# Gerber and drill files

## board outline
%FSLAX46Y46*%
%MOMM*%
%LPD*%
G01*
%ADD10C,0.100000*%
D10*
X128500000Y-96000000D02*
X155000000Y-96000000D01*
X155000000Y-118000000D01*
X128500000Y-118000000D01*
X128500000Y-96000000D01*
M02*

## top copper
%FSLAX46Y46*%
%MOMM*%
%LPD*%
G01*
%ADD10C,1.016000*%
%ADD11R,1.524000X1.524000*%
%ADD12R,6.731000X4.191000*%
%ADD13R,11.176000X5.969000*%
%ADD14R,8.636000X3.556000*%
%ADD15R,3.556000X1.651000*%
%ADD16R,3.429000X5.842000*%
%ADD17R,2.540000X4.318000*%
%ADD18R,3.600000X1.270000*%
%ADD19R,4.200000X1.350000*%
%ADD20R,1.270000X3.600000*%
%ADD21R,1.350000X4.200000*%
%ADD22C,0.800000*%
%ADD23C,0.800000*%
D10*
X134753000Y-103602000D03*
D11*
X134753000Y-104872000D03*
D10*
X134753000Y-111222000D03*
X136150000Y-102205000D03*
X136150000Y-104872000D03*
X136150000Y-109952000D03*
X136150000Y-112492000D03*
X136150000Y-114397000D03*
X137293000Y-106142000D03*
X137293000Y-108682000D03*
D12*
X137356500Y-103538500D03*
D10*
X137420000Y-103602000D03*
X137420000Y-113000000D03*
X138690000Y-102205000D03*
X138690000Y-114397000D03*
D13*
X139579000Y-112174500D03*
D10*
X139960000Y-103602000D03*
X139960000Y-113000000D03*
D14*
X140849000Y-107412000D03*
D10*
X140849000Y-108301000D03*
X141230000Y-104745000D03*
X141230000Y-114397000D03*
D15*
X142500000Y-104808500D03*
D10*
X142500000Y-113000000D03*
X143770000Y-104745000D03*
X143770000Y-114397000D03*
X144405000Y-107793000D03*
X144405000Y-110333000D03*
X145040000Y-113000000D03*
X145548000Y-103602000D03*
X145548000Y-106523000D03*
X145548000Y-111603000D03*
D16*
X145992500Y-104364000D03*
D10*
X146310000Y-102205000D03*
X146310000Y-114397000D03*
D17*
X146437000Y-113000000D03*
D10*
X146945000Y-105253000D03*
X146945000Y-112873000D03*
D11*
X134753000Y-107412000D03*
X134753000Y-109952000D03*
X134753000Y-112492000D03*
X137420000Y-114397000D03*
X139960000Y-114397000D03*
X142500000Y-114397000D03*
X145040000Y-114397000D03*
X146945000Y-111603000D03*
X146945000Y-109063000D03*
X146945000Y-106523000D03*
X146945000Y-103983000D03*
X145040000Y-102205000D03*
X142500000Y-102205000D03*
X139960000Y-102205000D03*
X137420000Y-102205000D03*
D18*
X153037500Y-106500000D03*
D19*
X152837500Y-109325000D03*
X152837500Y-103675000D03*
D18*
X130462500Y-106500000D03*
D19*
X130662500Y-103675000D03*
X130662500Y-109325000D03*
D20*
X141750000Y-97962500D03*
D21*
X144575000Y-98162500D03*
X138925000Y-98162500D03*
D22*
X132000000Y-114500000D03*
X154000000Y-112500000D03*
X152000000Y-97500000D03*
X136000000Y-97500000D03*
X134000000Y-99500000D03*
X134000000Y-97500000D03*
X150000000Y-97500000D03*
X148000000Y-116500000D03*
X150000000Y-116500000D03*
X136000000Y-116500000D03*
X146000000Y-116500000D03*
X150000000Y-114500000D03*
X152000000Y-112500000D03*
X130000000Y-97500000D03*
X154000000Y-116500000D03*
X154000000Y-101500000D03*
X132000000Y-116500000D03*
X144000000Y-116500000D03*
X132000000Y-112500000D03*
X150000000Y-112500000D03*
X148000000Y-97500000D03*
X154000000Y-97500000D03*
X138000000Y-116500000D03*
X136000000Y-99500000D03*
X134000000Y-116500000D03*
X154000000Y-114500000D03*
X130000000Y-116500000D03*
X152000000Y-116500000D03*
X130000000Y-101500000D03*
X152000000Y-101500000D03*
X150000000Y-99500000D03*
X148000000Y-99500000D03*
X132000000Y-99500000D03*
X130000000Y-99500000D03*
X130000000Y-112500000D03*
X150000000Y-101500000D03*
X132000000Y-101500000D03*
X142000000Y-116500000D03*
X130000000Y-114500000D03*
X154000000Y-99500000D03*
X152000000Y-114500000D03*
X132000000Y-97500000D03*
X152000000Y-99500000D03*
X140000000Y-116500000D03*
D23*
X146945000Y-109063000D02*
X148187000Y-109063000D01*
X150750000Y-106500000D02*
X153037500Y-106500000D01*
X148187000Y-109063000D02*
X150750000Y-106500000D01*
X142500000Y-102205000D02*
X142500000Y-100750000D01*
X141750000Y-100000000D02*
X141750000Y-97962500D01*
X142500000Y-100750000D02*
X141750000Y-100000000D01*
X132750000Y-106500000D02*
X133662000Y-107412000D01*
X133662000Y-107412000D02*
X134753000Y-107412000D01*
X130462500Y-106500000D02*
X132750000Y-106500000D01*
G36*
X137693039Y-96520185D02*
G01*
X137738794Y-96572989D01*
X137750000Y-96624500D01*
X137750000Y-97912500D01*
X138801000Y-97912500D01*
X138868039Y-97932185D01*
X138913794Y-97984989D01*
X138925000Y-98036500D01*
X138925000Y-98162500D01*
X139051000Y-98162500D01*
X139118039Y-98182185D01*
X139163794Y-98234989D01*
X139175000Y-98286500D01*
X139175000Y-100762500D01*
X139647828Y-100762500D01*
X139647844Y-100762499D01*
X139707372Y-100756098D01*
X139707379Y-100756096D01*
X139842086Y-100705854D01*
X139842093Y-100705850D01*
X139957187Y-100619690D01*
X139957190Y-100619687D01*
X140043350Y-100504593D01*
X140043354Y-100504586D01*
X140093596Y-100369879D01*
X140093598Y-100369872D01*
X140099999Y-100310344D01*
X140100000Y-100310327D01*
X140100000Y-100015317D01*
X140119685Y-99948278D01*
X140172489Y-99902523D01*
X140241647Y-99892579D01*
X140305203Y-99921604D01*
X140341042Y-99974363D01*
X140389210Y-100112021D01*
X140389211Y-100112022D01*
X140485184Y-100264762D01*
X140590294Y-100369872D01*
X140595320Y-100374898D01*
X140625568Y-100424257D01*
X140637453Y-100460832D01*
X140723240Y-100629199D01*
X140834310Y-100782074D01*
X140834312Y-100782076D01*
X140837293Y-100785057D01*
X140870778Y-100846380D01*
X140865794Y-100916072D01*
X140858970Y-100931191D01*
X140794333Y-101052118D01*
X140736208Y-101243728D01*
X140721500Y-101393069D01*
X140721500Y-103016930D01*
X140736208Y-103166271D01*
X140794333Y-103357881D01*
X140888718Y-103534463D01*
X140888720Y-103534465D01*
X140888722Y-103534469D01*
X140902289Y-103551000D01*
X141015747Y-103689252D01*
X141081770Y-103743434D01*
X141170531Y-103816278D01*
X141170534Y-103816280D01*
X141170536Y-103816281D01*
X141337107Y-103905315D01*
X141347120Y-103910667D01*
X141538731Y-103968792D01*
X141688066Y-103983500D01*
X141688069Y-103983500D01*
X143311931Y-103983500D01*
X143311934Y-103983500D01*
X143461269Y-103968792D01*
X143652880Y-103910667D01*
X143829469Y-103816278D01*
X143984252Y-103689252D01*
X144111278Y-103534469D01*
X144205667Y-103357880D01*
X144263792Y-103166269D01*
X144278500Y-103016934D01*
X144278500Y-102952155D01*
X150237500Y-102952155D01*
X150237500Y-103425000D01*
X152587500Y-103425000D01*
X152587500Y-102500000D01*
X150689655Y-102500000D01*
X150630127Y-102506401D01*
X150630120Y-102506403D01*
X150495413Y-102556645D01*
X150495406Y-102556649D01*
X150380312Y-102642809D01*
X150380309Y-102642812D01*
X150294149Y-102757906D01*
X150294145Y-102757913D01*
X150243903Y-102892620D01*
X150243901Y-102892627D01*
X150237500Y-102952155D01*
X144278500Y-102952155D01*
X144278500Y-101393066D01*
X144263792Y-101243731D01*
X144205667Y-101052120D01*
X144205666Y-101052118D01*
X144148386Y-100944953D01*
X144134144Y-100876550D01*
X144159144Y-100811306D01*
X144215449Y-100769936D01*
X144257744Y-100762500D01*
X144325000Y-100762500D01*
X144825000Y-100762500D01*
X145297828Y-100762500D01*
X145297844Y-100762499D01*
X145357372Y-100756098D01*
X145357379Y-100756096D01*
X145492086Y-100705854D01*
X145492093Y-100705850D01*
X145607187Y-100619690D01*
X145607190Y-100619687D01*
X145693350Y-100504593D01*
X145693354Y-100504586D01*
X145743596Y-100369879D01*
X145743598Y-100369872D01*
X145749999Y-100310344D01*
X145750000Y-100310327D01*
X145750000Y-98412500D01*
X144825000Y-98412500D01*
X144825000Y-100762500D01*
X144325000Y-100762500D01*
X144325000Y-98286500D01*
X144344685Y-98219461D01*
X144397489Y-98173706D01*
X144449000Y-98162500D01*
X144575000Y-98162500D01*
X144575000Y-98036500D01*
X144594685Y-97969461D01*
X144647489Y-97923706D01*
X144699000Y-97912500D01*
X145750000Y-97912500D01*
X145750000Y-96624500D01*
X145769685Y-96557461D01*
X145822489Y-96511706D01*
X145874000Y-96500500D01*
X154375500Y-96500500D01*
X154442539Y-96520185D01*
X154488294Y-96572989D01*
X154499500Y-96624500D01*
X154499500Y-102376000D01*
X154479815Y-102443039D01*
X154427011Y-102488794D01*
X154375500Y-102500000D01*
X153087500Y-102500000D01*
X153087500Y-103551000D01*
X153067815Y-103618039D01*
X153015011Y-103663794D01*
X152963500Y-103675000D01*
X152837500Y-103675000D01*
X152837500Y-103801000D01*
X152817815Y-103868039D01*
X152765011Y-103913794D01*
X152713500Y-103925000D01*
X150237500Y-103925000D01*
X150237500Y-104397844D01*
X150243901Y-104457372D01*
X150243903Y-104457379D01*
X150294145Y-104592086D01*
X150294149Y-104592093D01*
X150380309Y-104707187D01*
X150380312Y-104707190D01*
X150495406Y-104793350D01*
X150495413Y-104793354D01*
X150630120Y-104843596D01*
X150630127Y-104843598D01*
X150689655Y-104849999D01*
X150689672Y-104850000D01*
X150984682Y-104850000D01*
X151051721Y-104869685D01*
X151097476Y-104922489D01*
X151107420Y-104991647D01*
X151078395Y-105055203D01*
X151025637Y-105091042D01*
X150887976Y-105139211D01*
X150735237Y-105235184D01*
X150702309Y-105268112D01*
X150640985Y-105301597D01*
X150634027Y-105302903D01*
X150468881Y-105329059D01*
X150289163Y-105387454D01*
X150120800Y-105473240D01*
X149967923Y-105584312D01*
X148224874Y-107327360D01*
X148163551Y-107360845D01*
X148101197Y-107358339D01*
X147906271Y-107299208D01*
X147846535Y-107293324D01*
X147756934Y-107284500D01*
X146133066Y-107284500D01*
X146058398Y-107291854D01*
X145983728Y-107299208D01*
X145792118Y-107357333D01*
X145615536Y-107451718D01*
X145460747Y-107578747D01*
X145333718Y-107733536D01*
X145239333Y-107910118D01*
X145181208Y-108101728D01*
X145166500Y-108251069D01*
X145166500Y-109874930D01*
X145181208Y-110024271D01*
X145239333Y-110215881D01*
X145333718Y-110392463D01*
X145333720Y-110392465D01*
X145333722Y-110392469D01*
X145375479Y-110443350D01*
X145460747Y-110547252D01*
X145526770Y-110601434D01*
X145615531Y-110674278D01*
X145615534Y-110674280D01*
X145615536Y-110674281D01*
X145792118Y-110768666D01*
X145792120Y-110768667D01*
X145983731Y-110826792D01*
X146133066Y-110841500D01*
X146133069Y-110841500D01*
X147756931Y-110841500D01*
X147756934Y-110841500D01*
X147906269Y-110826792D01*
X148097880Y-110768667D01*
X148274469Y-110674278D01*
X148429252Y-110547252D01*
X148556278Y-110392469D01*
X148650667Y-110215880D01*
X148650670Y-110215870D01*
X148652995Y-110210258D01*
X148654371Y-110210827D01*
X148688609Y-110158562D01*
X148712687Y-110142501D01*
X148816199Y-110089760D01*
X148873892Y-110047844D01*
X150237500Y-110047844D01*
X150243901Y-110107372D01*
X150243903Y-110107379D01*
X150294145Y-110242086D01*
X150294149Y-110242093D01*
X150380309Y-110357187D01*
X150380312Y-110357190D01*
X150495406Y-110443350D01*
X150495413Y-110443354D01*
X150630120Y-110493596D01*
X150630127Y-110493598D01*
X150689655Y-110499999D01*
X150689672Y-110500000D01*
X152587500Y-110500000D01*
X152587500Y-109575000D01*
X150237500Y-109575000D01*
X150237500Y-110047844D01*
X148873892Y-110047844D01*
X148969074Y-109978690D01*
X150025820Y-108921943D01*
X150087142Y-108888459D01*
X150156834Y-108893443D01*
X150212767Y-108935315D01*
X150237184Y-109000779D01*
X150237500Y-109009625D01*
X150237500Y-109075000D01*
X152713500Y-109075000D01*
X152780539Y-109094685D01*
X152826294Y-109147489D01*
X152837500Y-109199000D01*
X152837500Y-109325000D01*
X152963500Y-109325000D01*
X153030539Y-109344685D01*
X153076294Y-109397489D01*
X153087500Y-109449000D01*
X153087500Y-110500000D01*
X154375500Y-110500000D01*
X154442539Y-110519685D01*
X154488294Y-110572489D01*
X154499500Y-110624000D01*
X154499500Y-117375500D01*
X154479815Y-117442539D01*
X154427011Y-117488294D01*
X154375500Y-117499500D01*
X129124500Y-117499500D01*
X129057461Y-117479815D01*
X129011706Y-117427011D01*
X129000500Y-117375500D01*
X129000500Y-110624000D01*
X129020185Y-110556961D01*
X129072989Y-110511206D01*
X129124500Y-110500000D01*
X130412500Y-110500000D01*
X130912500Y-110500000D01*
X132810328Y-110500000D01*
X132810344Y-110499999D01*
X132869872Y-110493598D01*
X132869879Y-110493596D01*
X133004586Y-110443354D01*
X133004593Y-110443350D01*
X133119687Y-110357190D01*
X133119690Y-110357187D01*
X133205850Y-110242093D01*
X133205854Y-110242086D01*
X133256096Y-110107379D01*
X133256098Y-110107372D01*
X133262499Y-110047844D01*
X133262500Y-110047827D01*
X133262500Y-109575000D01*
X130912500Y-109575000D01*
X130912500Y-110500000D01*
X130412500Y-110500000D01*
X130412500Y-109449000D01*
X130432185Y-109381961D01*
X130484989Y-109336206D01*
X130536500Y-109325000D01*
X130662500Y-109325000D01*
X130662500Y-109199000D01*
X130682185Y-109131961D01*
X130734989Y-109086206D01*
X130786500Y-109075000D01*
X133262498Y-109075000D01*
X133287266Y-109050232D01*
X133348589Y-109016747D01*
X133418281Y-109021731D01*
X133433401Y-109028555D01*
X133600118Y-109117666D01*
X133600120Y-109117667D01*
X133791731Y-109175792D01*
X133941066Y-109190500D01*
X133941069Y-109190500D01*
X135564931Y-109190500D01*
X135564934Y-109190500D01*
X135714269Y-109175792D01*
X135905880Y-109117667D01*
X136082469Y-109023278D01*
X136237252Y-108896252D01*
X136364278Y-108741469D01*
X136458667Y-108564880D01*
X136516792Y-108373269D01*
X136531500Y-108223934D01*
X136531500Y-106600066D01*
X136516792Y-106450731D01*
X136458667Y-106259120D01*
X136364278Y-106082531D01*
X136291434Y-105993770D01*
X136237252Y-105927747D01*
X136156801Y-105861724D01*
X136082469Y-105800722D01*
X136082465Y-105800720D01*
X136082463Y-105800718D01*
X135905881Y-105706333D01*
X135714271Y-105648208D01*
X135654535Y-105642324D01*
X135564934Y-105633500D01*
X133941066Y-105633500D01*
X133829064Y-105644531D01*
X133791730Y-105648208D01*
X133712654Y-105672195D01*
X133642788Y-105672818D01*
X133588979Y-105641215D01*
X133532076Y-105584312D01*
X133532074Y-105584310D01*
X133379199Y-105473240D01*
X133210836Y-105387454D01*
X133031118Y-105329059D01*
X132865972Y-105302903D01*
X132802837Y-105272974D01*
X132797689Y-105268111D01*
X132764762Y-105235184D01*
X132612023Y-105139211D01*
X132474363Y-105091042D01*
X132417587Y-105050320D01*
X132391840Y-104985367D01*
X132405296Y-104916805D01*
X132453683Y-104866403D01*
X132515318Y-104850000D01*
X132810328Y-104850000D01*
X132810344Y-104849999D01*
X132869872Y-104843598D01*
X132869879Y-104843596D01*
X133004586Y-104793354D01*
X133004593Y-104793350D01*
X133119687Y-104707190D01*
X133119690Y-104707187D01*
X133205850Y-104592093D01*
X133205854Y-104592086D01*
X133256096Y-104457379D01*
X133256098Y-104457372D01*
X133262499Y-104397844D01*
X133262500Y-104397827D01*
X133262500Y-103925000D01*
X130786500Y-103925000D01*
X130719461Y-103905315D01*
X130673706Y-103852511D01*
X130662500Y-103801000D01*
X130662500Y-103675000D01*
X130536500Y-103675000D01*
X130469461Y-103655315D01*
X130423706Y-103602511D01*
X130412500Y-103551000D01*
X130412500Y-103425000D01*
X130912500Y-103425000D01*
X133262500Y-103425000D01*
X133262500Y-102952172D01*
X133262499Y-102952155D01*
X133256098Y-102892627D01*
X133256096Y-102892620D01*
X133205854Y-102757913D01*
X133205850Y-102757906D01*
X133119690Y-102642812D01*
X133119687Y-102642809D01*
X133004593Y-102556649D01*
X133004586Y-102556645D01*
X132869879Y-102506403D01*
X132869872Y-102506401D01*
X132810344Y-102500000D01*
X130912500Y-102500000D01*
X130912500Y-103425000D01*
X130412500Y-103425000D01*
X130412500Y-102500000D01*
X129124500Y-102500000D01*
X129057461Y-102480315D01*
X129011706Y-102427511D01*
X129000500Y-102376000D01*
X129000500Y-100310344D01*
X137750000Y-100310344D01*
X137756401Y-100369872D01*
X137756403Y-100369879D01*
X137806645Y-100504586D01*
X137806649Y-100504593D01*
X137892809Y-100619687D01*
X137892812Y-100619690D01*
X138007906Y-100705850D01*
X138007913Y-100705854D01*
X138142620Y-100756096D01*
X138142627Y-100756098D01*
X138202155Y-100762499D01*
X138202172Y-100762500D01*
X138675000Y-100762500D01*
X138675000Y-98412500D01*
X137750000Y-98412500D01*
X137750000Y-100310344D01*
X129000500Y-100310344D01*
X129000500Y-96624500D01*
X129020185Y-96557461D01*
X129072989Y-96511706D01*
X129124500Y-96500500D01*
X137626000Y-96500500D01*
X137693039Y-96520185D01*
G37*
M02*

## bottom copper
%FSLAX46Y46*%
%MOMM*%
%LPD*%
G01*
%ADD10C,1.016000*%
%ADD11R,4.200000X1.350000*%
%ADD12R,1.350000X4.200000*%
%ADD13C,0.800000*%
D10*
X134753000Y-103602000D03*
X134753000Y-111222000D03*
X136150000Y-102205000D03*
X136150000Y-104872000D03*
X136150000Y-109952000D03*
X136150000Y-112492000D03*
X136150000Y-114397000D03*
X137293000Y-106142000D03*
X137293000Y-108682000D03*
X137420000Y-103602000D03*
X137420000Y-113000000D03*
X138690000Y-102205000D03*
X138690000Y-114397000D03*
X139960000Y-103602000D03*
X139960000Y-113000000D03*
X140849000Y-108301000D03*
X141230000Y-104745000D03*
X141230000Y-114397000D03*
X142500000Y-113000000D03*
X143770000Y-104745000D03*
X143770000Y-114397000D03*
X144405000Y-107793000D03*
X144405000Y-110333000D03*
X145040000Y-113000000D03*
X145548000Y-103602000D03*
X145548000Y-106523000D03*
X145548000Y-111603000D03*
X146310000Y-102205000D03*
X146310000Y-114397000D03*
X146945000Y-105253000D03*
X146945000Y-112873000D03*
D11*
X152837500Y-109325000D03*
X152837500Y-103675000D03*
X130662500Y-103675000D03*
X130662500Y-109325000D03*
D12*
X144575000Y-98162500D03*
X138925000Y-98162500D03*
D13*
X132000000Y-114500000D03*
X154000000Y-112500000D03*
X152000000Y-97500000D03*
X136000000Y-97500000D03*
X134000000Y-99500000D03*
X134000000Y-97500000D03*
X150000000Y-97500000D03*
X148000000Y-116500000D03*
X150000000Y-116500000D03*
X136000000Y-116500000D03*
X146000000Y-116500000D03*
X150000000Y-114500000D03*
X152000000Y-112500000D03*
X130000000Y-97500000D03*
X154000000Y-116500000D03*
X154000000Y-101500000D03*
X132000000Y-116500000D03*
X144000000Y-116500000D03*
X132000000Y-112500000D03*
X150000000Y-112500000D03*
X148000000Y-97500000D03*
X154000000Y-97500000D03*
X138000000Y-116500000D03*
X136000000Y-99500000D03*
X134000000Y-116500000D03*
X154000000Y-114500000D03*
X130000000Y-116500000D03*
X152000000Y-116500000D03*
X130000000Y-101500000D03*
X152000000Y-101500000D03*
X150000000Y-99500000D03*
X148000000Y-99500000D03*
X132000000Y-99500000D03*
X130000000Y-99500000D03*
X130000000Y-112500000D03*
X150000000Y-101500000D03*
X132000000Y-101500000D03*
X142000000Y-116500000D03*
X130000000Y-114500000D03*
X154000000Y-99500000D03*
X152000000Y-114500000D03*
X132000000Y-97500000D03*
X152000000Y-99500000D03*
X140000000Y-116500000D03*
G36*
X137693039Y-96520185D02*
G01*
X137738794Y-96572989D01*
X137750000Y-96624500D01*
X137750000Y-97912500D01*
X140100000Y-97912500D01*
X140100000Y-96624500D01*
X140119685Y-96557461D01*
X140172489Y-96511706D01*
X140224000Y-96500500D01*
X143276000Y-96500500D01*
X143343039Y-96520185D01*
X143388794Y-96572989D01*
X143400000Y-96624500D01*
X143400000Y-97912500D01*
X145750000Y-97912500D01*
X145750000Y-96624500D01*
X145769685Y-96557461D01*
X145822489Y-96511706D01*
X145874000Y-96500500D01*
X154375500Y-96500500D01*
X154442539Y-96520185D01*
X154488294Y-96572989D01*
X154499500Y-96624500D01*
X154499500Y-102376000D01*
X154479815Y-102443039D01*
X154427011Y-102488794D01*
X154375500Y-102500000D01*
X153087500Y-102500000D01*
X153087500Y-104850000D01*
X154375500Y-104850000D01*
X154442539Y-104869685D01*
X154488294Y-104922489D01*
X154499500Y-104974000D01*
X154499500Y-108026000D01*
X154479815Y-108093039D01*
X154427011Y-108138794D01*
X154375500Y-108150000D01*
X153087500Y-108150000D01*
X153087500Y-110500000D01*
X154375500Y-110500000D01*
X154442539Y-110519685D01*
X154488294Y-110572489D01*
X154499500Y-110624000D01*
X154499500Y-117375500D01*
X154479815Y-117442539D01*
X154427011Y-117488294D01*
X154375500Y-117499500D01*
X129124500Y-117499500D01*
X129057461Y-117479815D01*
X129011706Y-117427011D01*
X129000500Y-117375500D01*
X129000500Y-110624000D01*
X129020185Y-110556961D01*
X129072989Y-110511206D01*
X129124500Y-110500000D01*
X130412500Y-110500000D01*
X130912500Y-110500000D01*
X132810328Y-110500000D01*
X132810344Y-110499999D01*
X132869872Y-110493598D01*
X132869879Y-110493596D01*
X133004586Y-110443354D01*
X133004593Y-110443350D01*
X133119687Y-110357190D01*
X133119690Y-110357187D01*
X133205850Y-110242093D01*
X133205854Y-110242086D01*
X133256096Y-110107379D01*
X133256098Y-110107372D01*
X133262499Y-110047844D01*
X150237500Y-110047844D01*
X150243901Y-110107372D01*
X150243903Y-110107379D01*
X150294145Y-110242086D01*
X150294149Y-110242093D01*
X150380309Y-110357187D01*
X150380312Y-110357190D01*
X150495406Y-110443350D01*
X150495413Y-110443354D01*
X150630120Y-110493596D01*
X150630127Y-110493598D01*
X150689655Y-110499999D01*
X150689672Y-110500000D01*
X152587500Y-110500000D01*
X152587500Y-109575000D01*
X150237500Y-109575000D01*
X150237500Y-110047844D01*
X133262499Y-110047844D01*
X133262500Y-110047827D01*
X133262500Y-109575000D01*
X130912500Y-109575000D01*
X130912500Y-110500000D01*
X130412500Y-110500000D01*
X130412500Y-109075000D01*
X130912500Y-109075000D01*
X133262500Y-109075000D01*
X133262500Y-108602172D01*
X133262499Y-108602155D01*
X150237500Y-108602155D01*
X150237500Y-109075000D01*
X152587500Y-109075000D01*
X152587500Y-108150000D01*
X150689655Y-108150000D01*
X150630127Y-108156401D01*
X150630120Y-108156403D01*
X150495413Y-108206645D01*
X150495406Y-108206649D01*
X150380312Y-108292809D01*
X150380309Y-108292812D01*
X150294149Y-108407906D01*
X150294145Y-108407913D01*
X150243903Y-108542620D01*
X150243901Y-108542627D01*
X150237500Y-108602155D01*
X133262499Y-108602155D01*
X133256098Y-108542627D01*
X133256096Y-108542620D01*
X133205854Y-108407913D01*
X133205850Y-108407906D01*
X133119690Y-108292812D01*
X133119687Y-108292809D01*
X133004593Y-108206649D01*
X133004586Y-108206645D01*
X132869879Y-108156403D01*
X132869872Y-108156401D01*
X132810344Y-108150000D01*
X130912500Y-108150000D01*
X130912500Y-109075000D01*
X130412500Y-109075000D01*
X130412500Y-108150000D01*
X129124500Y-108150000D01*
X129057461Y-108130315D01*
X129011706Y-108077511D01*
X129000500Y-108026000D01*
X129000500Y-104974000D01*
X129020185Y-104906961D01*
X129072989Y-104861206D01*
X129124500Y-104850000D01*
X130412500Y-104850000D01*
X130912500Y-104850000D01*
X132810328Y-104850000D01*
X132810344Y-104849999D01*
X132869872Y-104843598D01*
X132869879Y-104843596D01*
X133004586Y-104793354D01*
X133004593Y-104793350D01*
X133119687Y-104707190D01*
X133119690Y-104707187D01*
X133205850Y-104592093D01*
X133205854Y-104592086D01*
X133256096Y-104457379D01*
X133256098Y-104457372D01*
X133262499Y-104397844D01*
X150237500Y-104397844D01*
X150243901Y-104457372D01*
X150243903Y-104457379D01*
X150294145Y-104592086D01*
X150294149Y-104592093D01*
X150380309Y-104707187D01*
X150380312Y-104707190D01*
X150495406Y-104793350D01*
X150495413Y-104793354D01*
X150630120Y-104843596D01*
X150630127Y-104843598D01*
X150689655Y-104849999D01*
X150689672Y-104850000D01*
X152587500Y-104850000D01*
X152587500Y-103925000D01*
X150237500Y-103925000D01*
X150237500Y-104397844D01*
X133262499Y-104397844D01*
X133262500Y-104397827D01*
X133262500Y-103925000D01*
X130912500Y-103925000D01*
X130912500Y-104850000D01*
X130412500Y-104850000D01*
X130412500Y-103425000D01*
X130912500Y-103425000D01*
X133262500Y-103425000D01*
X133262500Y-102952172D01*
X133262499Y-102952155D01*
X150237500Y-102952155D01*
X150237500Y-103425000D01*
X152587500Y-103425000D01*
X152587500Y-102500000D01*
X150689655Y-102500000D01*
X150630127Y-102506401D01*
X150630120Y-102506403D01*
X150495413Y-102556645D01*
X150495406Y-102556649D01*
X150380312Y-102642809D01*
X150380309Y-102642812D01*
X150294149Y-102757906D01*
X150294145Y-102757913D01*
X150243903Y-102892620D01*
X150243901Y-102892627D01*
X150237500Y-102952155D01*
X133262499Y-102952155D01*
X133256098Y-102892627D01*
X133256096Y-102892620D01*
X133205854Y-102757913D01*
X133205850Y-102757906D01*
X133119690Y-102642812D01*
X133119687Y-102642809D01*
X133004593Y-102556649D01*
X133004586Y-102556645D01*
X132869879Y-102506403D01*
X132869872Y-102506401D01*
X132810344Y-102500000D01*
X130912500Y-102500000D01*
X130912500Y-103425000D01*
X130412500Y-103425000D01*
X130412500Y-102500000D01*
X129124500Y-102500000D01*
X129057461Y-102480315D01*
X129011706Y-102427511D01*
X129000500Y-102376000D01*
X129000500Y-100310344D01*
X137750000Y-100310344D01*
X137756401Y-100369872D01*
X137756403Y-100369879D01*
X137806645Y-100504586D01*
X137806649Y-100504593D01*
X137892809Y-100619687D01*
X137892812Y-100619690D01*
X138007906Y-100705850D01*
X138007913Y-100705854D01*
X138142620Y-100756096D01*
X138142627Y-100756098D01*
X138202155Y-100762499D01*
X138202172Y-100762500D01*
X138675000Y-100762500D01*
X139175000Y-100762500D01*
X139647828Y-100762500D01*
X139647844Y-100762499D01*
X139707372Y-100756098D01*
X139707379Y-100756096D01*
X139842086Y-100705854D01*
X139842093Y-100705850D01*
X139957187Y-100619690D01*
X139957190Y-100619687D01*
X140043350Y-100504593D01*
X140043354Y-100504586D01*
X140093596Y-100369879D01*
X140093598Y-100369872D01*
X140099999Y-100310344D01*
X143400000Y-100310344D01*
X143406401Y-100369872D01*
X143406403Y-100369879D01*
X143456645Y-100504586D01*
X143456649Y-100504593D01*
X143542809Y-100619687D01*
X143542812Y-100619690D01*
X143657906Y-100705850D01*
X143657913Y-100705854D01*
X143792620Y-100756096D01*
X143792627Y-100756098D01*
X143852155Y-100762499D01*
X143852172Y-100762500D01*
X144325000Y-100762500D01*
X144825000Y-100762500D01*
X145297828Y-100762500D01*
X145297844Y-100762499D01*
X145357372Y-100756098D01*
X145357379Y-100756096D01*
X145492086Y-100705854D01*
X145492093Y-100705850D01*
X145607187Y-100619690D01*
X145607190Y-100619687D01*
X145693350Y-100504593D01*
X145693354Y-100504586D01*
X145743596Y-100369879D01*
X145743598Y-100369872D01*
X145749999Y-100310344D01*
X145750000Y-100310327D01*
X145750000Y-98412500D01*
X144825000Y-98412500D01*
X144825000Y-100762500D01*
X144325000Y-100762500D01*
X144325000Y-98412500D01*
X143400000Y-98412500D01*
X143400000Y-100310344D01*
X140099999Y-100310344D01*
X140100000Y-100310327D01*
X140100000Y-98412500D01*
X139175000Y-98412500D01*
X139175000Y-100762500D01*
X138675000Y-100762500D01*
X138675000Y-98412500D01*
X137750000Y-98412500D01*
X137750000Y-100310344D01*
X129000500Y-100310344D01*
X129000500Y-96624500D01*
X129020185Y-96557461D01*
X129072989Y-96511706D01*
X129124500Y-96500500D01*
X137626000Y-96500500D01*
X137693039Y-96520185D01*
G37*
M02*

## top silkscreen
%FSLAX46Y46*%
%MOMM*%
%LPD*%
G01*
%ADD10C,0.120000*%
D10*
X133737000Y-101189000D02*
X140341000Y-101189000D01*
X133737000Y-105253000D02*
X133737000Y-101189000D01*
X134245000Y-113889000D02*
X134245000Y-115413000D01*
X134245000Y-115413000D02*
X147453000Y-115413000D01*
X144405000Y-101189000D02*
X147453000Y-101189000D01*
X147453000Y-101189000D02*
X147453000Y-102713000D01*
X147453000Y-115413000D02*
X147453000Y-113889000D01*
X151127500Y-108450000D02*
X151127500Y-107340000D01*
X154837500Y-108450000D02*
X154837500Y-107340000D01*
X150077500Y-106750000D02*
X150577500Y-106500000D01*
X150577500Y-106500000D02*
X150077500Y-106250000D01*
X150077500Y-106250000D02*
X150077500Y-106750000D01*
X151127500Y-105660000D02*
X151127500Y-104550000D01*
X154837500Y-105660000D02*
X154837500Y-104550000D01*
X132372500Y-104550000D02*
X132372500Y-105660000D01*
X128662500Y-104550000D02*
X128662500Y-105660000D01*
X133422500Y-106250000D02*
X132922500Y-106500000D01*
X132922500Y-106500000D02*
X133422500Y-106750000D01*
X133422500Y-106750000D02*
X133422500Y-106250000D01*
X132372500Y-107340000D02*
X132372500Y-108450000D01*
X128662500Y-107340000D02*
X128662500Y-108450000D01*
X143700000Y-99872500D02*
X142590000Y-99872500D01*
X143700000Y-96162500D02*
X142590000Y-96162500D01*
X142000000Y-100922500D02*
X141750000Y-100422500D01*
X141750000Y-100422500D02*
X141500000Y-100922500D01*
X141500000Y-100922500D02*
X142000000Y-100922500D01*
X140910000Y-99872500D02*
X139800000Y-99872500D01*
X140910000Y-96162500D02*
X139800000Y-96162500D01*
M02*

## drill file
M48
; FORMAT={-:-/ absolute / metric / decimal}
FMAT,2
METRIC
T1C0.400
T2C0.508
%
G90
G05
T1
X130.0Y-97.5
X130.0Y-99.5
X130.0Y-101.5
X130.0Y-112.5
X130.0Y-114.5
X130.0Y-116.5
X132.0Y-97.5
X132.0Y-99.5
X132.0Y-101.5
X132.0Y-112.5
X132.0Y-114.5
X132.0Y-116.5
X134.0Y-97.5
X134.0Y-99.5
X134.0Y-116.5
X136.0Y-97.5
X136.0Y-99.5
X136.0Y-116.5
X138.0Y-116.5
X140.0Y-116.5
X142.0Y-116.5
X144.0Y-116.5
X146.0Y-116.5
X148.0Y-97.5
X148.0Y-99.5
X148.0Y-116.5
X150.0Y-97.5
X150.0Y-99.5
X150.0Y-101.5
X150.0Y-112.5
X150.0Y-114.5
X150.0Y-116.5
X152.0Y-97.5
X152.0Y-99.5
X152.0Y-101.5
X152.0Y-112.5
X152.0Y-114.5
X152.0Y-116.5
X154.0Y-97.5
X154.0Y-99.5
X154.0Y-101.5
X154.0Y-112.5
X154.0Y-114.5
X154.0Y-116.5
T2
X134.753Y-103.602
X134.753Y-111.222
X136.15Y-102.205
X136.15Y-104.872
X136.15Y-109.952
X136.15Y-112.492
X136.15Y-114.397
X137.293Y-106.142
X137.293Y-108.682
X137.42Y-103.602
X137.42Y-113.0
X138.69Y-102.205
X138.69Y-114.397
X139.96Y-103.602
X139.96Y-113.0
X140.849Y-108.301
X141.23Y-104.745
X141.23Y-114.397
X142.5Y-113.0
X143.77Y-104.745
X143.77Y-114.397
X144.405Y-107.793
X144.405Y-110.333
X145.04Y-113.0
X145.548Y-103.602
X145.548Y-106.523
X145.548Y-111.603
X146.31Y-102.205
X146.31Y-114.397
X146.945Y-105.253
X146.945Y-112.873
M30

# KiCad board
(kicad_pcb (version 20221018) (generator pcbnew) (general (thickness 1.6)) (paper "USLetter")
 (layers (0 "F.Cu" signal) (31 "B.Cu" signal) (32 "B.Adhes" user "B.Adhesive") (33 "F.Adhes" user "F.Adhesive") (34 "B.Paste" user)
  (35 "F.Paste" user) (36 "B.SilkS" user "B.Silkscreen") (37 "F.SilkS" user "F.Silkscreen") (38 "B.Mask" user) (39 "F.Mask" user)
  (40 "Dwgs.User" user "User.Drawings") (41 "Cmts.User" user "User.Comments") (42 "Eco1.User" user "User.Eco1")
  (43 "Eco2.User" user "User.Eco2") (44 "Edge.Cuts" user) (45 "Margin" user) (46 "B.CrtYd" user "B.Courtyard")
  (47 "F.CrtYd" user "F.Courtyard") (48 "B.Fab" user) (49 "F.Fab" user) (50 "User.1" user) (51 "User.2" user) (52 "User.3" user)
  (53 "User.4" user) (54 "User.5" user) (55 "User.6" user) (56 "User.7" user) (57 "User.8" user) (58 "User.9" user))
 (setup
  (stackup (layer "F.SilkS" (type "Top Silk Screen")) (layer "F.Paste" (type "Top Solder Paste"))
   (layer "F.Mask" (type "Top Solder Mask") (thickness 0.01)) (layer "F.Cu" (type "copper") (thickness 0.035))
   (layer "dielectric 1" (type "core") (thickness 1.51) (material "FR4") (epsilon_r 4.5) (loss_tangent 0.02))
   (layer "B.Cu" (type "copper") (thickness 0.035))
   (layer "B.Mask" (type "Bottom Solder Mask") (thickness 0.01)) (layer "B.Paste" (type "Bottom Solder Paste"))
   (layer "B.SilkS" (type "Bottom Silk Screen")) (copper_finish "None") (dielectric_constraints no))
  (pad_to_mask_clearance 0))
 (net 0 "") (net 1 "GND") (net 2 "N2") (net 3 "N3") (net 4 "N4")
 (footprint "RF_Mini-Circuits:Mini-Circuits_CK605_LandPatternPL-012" (layer "F.Cu") (at 140.849 108.301)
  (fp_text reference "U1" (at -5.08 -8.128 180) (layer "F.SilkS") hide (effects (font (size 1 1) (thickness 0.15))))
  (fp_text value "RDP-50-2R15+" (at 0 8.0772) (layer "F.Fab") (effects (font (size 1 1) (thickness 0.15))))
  (fp_line (start -7.112 -7.112) (end -0.508 -7.112) (stroke (width 0.12) (type solid)) (layer "F.SilkS"))
  (fp_line (start -7.112 -3.048) (end -7.112 -7.112) (stroke (width 0.12) (type solid)) (layer "F.SilkS"))
  (fp_line (start -6.604 5.588) (end -6.604 7.112) (stroke (width 0.12) (type solid)) (layer "F.SilkS"))
  (fp_line (start -6.604 7.112) (end 6.604 7.112) (stroke (width 0.12) (type solid)) (layer "F.SilkS"))
  (fp_line (start 3.556 -7.112) (end 6.604 -7.112) (stroke (width 0.12) (type solid)) (layer "F.SilkS"))
  (fp_line (start 6.604 -7.112) (end 6.604 -5.588) (stroke (width 0.12) (type solid)) (layer "F.SilkS"))
  (fp_line (start 6.604 7.112) (end 6.604 5.588) (stroke (width 0.12) (type solid)) (layer "F.SilkS"))
  (pad "1" thru_hole circle (at -6.096 -4.699) (size 1.016 1.016) (drill 0.508) (layers "*.Cu") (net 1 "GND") (zone_connect 2))
  (pad "1" smd rect (at -6.096 -3.429 270) (size 1.524 1.524) (layers "F.Cu" "F.Paste" "F.Mask") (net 1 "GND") (zone_connect 2))
  (pad "1" thru_hole circle (at -6.096 2.921) (size 1.016 1.016) (drill 0.508) (layers "*.Cu") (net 1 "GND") (zone_connect 2))
  (pad "1" thru_hole circle (at -4.699 -6.096) (size 1.016 1.016) (drill 0.508) (layers "*.Cu") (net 1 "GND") (zone_connect 2))
  (pad "1" thru_hole circle (at -4.699 -3.429) (size 1.016 1.016) (drill 0.508) (layers "*.Cu") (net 1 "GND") (zone_connect 2))
  (pad "1" thru_hole circle (at -4.699 1.651) (size 1.016 1.016) (drill 0.508) (layers "*.Cu") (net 1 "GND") (zone_connect 2))
  (pad "1" thru_hole circle (at -4.699 4.191) (size 1.016 1.016) (drill 0.508) (layers "*.Cu") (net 1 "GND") (zone_connect 2))
  (pad "1" thru_hole circle (at -4.699 6.096) (size 1.016 1.016) (drill 0.508) (layers "*.Cu") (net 1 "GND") (zone_connect 2))
  (pad "1" thru_hole circle (at -3.556 -2.159) (size 1.016 1.016) (drill 0.508) (layers "*.Cu") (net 1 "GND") (zone_connect 2))
  (pad "1" thru_hole circle (at -3.556 0.381) (size 1.016 1.016) (drill 0.508) (layers "*.Cu") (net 1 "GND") (zone_connect 2))
  (pad "1" smd rect (at -3.4925 -4.7625) (size 6.731 4.191) (layers "F.Cu") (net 1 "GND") (zone_connect 2))
  (pad "1" thru_hole circle (at -3.429 -4.699) (size 1.016 1.016) (drill 0.508) (layers "*.Cu") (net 1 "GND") (zone_connect 2))
  (pad "1" thru_hole circle (at -3.429 4.699) (size 1.016 1.016) (drill 0.508) (layers "*.Cu") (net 1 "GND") (zone_connect 2))
  (pad "1" thru_hole circle (at -2.159 -6.096) (size 1.016 1.016) (drill 0.508) (layers "*.Cu") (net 1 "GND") (zone_connect 2))
  (pad "1" thru_hole circle (at -2.159 6.096) (size 1.016 1.016) (drill 0.508) (layers "*.Cu") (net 1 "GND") (zone_connect 2))
  (pad "1" smd rect (at -1.27 3.8735) (size 11.176 5.969) (layers "F.Cu") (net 1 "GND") (zone_connect 2))
  (pad "1" thru_hole circle (at -0.889 -4.699) (size 1.016 1.016) (drill 0.508) (layers "*.Cu") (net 1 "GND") (zone_connect 2))
  (pad "1" thru_hole circle (at -0.889 4.699) (size 1.016 1.016) (drill 0.508) (layers "*.Cu") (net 1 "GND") (zone_connect 2))
  (pad "1" smd rect (at 0 -0.889) (size 8.636 3.556) (layers "F.Cu") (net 1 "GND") (zone_connect 2))
  (pad "1" thru_hole circle (at 0 0) (size 1.016 1.016) (drill 0.508) (layers "*.Cu") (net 1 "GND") (zone_connect 2))
  (pad "1" thru_hole circle (at 0.381 -3.556) (size 1.016 1.016) (drill 0.508) (layers "*.Cu") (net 1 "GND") (zone_connect 2))
  (pad "1" thru_hole circle (at 0.381 6.096) (size 1.016 1.016) (drill 0.508) (layers "*.Cu") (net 1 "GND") (zone_connect 2))
  (pad "1" smd rect (at 1.651 -3.4925) (size 3.556 1.651) (layers "F.Cu") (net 1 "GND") (zone_connect 2))
  (pad "1" thru_hole circle (at 1.651 4.699) (size 1.016 1.016) (drill 0.508) (layers "*.Cu") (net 1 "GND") (zone_connect 2))
  (pad "1" thru_hole circle (at 2.921 -3.556) (size 1.016 1.016) (drill 0.508) (layers "*.Cu") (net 1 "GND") (zone_connect 2))
  (pad "1" thru_hole circle (at 2.921 6.096) (size 1.016 1.016) (drill 0.508) (layers "*.Cu") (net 1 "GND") (zone_connect 2))
  (pad "1" thru_hole circle (at 3.556 -0.508) (size 1.016 1.016) (drill 0.508) (layers "*.Cu") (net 1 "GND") (zone_connect 2))
  (pad "1" thru_hole circle (at 3.556 2.032) (size 1.016 1.016) (drill 0.508) (layers "*.Cu") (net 1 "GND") (zone_connect 2))
  (pad "1" thru_hole circle (at 4.191 4.699) (size 1.016 1.016) (drill 0.508) (layers "*.Cu") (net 1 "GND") (zone_connect 2))
  (pad "1" thru_hole circle (at 4.699 -4.699) (size 1.016 1.016) (drill 0.508) (layers "*.Cu") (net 1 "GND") (zone_connect 2))
  (pad "1" thru_hole circle (at 4.699 -1.778) (size 1.016 1.016) (drill 0.508) (layers "*.Cu") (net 1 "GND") (zone_connect 2))
  (pad "1" thru_hole circle (at 4.699 3.302) (size 1.016 1.016) (drill 0.508) (layers "*.Cu") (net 1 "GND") (zone_connect 2))
  (pad "1" smd rect (at 5.1435 -3.937) (size 3.429 5.842) (layers "F.Cu") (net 1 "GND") (zone_connect 2))
  (pad "1" thru_hole circle (at 5.461 -6.096) (size 1.016 1.016) (drill 0.508) (layers "*.Cu") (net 1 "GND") (zone_connect 2))
  (pad "1" thru_hole circle (at 5.461 6.096) (size 1.016 1.016) (drill 0.508) (layers "*.Cu") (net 1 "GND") (zone_connect 2))
  (pad "1" smd rect (at 5.588 4.699) (size 2.54 4.318) (layers "F.Cu") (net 1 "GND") (zone_connect 2))
  (pad "1" thru_hole circle (at 6.096 -3.048) (size 1.016 1.016) (drill 0.508) (layers "*.Cu") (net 1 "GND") (zone_connect 2))
  (pad "1" thru_hole circle (at 6.096 4.572) (size 1.016 1.016) (drill 0.508) (layers "*.Cu") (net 1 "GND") (zone_connect 2))
  (pad "2" smd rect (at -6.096 -0.889 270) (size 1.524 1.524) (layers "F.Cu" "F.Paste" "F.Mask") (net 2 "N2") (clearance 1.016))
  (pad "3" smd rect (at -6.096 1.651 270) (size 1.524 1.524) (layers "F.Cu" "F.Paste" "F.Mask") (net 1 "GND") (zone_connect 2))
  (pad "4" smd rect (at -6.096 4.191 270) (size 1.524 1.524) (layers "F.Cu" "F.Paste" "F.Mask") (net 1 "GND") (zone_connect 2))
  (pad "5" smd rect (at -3.429 6.096 270) (size 1.524 1.524) (layers "F.Cu" "F.Paste" "F.Mask") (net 1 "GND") (zone_connect 2))
  (pad "6" smd rect (at -0.889 6.096 270) (size 1.524 1.524) (layers "F.Cu" "F.Paste" "F.Mask") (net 1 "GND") (zone_connect 2))
  (pad "7" smd rect (at 1.651 6.096 270) (size 1.524 1.524) (layers "F.Cu" "F.Paste" "F.Mask") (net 1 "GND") (zone_connect 2))
  (pad "8" smd rect (at 4.191 6.096 270) (size 1.524 1.524) (layers "F.Cu" "F.Paste" "F.Mask") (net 1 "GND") (zone_connect 2))
  (pad "9" smd rect (at 6.096 3.302 270) (size 1.524 1.524) (layers "F.Cu" "F.Paste" "F.Mask") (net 1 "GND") (zone_connect 2))
  (pad "10" smd rect (at 6.096 0.762 270) (size 1.524 1.524) (layers "F.Cu" "F.Paste" "F.Mask") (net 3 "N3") (clearance 1.016))
  (pad "11" smd rect (at 6.096 -1.778 270) (size 1.524 1.524) (layers "F.Cu" "F.Paste" "F.Mask") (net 1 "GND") (zone_connect 2))
  (pad "12" smd rect (at 6.096 -4.318 270) (size 1.524 1.524) (layers "F.Cu" "F.Paste" "F.Mask") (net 1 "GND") (zone_connect 2))
  (pad "13" smd rect (at 4.191 -6.096 270) (size 1.524 1.524) (layers "F.Cu" "F.Paste" "F.Mask") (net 1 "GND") (zone_connect 2))
  (pad "14" smd rect (at 1.651 -6.096 270) (size 1.524 1.524) (layers "F.Cu" "F.Paste" "F.Mask") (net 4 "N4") (clearance 1.016))
  (pad "15" smd rect (at -0.889 -6.096 270) (size 1.524 1.524) (layers "F.Cu" "F.Paste" "F.Mask") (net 1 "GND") (zone_connect 2))
  (pad "16" smd rect (at -3.429 -6.096 270) (size 1.524 1.524) (layers "F.Cu" "F.Paste" "F.Mask") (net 1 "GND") (zone_connect 2)))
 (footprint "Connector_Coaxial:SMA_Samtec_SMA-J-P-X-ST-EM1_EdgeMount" (layer "F.Cu") (at 152.8375 106.5 90)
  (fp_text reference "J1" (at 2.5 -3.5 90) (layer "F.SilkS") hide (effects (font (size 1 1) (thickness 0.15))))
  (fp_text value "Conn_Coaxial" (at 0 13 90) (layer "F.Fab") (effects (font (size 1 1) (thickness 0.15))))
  (fp_line (start -1.95 -1.71) (end -0.84 -1.71) (stroke (width 0.12) (type solid)) (layer "F.SilkS"))
  (fp_line (start -1.95 2) (end -0.84 2) (stroke (width 0.12) (type solid)) (layer "F.SilkS"))
  (fp_line (start -0.25 -2.76) (end 0 -2.26) (stroke (width 0.12) (type solid)) (layer "F.SilkS"))
  (fp_line (start 0 -2.26) (end 0.25 -2.76) (stroke (width 0.12) (type solid)) (layer "F.SilkS"))
  (fp_line (start 0.25 -2.76) (end -0.25 -2.76) (stroke (width 0.12) (type solid)) (layer "F.SilkS"))
  (fp_line (start 0.84 -1.71) (end 1.95 -1.71) (stroke (width 0.12) (type solid)) (layer "F.SilkS"))
  (fp_line (start 0.84 2) (end 1.95 2) (stroke (width 0.12) (type solid)) (layer "F.SilkS"))
  (pad "1" smd rect (at 0 0.2 90) (size 1.27 3.6) (layers "F.Cu" "F.Paste" "F.Mask") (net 3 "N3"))
  (pad "2" smd rect (at -2.825 0 90) (size 1.35 4.2) (layers "F.Cu" "F.Paste" "F.Mask") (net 1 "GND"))
  (pad "2" smd rect (at -2.825 0 90) (size 1.35 4.2) (layers "B.Cu" "B.Paste" "B.Mask") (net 1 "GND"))
  (pad "2" smd rect (at 2.825 0 90) (size 1.35 4.2) (layers "F.Cu" "F.Paste" "F.Mask") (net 1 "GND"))
  (pad "2" smd rect (at 2.825 0 90) (size 1.35 4.2) (layers "B.Cu" "B.Paste" "B.Mask") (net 1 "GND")))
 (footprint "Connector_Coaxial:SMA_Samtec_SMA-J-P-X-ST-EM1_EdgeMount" (layer "F.Cu") (at 130.6625 106.5 -90)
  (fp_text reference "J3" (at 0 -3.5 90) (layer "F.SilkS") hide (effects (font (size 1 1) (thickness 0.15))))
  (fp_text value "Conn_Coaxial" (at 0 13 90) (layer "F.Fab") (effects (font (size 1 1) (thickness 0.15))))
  (fp_line (start -1.95 -1.71) (end -0.84 -1.71) (stroke (width 0.12) (type solid)) (layer "F.SilkS"))
  (fp_line (start -1.95 2) (end -0.84 2) (stroke (width 0.12) (type solid)) (layer "F.SilkS"))
  (fp_line (start -0.25 -2.76) (end 0 -2.26) (stroke (width 0.12) (type solid)) (layer "F.SilkS"))
  (fp_line (start 0 -2.26) (end 0.25 -2.76) (stroke (width 0.12) (type solid)) (layer "F.SilkS"))
  (fp_line (start 0.25 -2.76) (end -0.25 -2.76) (stroke (width 0.12) (type solid)) (layer "F.SilkS"))
  (fp_line (start 0.84 -1.71) (end 1.95 -1.71) (stroke (width 0.12) (type solid)) (layer "F.SilkS"))
  (fp_line (start 0.84 2) (end 1.95 2) (stroke (width 0.12) (type solid)) (layer "F.SilkS"))
  (pad "1" smd rect (at 0 0.2 270) (size 1.27 3.6) (layers "F.Cu" "F.Paste" "F.Mask") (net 2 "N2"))
  (pad "2" smd rect (at -2.825 0 270) (size 1.35 4.2) (layers "F.Cu" "F.Paste" "F.Mask") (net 1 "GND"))
  (pad "2" smd rect (at -2.825 0 270) (size 1.35 4.2) (layers "B.Cu" "B.Paste" "B.Mask") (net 1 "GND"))
  (pad "2" smd rect (at 2.825 0 270) (size 1.35 4.2) (layers "F.Cu" "F.Paste" "F.Mask") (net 1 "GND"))
  (pad "2" smd rect (at 2.825 0 270) (size 1.35 4.2) (layers "B.Cu" "B.Paste" "B.Mask") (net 1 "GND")))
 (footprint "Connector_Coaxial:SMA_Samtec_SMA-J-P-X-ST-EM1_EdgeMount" (layer "F.Cu") (at 141.75 98.1625 180)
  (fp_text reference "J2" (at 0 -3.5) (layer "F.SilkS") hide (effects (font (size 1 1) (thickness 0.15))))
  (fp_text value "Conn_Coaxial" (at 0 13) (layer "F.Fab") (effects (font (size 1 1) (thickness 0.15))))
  (fp_line (start -1.95 -1.71) (end -0.84 -1.71) (stroke (width 0.12) (type solid)) (layer "F.SilkS"))
  (fp_line (start -1.95 2) (end -0.84 2) (stroke (width 0.12) (type solid)) (layer "F.SilkS"))
  (fp_line (start -0.25 -2.76) (end 0 -2.26) (stroke (width 0.12) (type solid)) (layer "F.SilkS"))
  (fp_line (start 0 -2.26) (end 0.25 -2.76) (stroke (width 0.12) (type solid)) (layer "F.SilkS"))
  (fp_line (start 0.25 -2.76) (end -0.25 -2.76) (stroke (width 0.12) (type solid)) (layer "F.SilkS"))
  (fp_line (start 0.84 -1.71) (end 1.95 -1.71) (stroke (width 0.12) (type solid)) (layer "F.SilkS"))
  (fp_line (start 0.84 2) (end 1.95 2) (stroke (width 0.12) (type solid)) (layer "F.SilkS"))
  (pad "1" smd rect (at 0 0.2 180) (size 1.27 3.6) (layers "F.Cu" "F.Paste" "F.Mask") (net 4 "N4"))
  (pad "2" smd rect (at -2.825 0 180) (size 1.35 4.2) (layers "F.Cu" "F.Paste" "F.Mask") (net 1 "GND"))
  (pad "2" smd rect (at -2.825 0 180) (size 1.35 4.2) (layers "B.Cu" "B.Paste" "B.Mask") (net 1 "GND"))
  (pad "2" smd rect (at 2.825 0 180) (size 1.35 4.2) (layers "F.Cu" "F.Paste" "F.Mask") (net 1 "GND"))
  (pad "2" smd rect (at 2.825 0 180) (size 1.35 4.2) (layers "B.Cu" "B.Paste" "B.Mask") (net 1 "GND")))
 (gr_rect (start 128.5 96) (end 155 118) (stroke (width 0.1) (type default)) (fill none) (layer "Edge.Cuts"))
 (segment (start 146.945 109.063) (end 148.187 109.063) (width 0.8) (layer "F.Cu") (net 3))
 (segment (start 150.75 106.5) (end 153.0375 106.5) (width 0.8) (layer "F.Cu") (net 3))
 (segment (start 148.187 109.063) (end 150.75 106.5) (width 0.8) (layer "F.Cu") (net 3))
 (segment (start 142.5 102.205) (end 142.5 100.75) (width 0.8) (layer "F.Cu") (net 4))
 (segment (start 141.75 100) (end 141.75 97.9625) (width 0.8) (layer "F.Cu") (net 4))
 (segment (start 142.5 100.75) (end 141.75 100) (width 0.8) (layer "F.Cu") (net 4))
 (via (at 132 114.5) (size 0.8) (drill 0.4) (layers "F.Cu" "B.Cu") (free) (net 1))
 (via (at 154 112.5) (size 0.8) (drill 0.4) (layers "F.Cu" "B.Cu") (free) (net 1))
 (via (at 152 97.5) (size 0.8) (drill 0.4) (layers "F.Cu" "B.Cu") (free) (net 1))
 (via (at 136 97.5) (size 0.8) (drill 0.4) (layers "F.Cu" "B.Cu") (free) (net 1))
 (via (at 134 99.5) (size 0.8) (drill 0.4) (layers "F.Cu" "B.Cu") (free) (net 1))
 (via (at 134 97.5) (size 0.8) (drill 0.4) (layers "F.Cu" "B.Cu") (free) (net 1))
 (via (at 150 97.5) (size 0.8) (drill 0.4) (layers "F.Cu" "B.Cu") (free) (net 1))
 (via (at 148 116.5) (size 0.8) (drill 0.4) (layers "F.Cu" "B.Cu") (free) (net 1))
 (via (at 150 116.5) (size 0.8) (drill 0.4) (layers "F.Cu" "B.Cu") (free) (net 1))
 (via (at 136 116.5) (size 0.8) (drill 0.4) (layers "F.Cu" "B.Cu") (free) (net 1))
 (via (at 146 116.5) (size 0.8) (drill 0.4) (layers "F.Cu" "B.Cu") (free) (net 1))
 (via (at 150 114.5) (size 0.8) (drill 0.4) (layers "F.Cu" "B.Cu") (free) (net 1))
 (via (at 152 112.5) (size 0.8) (drill 0.4) (layers "F.Cu" "B.Cu") (free) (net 1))
 (via (at 130 97.5) (size 0.8) (drill 0.4) (layers "F.Cu" "B.Cu") (free) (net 1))
 (via (at 154 116.5) (size 0.8) (drill 0.4) (layers "F.Cu" "B.Cu") (free) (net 1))
 (via (at 154 101.5) (size 0.8) (drill 0.4) (layers "F.Cu" "B.Cu") (free) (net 1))
 (via (at 132 116.5) (size 0.8) (drill 0.4) (layers "F.Cu" "B.Cu") (free) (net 1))
 (via (at 144 116.5) (size 0.8) (drill 0.4) (layers "F.Cu" "B.Cu") (free) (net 1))
 (via (at 132 112.5) (size 0.8) (drill 0.4) (layers "F.Cu" "B.Cu") (free) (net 1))
 (via (at 150 112.5) (size 0.8) (drill 0.4) (layers "F.Cu" "B.Cu") (free) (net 1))
 (via (at 148 97.5) (size 0.8) (drill 0.4) (layers "F.Cu" "B.Cu") (free) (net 1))
 (via (at 154 97.5) (size 0.8) (drill 0.4) (layers "F.Cu" "B.Cu") (free) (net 1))
 (via (at 138 116.5) (size 0.8) (drill 0.4) (layers "F.Cu" "B.Cu") (free) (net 1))
 (via (at 136 99.5) (size 0.8) (drill 0.4) (layers "F.Cu" "B.Cu") (free) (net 1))
 (via (at 134 116.5) (size 0.8) (drill 0.4) (layers "F.Cu" "B.Cu") (free) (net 1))
 (via (at 154 114.5) (size 0.8) (drill 0.4) (layers "F.Cu" "B.Cu") (free) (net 1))
 (via (at 130 116.5) (size 0.8) (drill 0.4) (layers "F.Cu" "B.Cu") (free) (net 1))
 (via (at 152 116.5) (size 0.8) (drill 0.4) (layers "F.Cu" "B.Cu") (free) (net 1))
 (via (at 130 101.5) (size 0.8) (drill 0.4) (layers "F.Cu" "B.Cu") (free) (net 1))
 (via (at 152 101.5) (size 0.8) (drill 0.4) (layers "F.Cu" "B.Cu") (free) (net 1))
 (via (at 150 99.5) (size 0.8) (drill 0.4) (layers "F.Cu" "B.Cu") (free) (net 1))
 (via (at 148 99.5) (size 0.8) (drill 0.4) (layers "F.Cu" "B.Cu") (free) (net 1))
 (via (at 132 99.5) (size 0.8) (drill 0.4) (layers "F.Cu" "B.Cu") (free) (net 1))
 (via (at 130 99.5) (size 0.8) (drill 0.4) (layers "F.Cu" "B.Cu") (free) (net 1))
 (via (at 130 112.5) (size 0.8) (drill 0.4) (layers "F.Cu" "B.Cu") (free) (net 1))
 (via (at 150 101.5) (size 0.8) (drill 0.4) (layers "F.Cu" "B.Cu") (free) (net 1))
 (via (at 132 101.5) (size 0.8) (drill 0.4) (layers "F.Cu" "B.Cu") (free) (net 1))
 (via (at 142 116.5) (size 0.8) (drill 0.4) (layers "F.Cu" "B.Cu") (free) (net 1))
 (via (at 130 114.5) (size 0.8) (drill 0.4) (layers "F.Cu" "B.Cu") (free) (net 1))
 (via (at 154 99.5) (size 0.8) (drill 0.4) (layers "F.Cu" "B.Cu") (free) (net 1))
 (via (at 152 114.5) (size 0.8) (drill 0.4) (layers "F.Cu" "B.Cu") (free) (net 1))
 (via (at 132 97.5) (size 0.8) (drill 0.4) (layers "F.Cu" "B.Cu") (free) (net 1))
 (via (at 152 99.5) (size 0.8) (drill 0.4) (layers "F.Cu" "B.Cu") (free) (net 1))
 (via (at 140 116.5) (size 0.8) (drill 0.4) (layers "F.Cu" "B.Cu") (free) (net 1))
 (segment (start 132.75 106.5) (end 133.662 107.412) (width 0.8) (layer "F.Cu") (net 2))
 (segment (start 133.662 107.412) (end 134.753 107.412) (width 0.8) (layer "F.Cu") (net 2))
 (segment (start 130.4625 106.5) (end 132.75 106.5) (width 0.8) (layer "F.Cu") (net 2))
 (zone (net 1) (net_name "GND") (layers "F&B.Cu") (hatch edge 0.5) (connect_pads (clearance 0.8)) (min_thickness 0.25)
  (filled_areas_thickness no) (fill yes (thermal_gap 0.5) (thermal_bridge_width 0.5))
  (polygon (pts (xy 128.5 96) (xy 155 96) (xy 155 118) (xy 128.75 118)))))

